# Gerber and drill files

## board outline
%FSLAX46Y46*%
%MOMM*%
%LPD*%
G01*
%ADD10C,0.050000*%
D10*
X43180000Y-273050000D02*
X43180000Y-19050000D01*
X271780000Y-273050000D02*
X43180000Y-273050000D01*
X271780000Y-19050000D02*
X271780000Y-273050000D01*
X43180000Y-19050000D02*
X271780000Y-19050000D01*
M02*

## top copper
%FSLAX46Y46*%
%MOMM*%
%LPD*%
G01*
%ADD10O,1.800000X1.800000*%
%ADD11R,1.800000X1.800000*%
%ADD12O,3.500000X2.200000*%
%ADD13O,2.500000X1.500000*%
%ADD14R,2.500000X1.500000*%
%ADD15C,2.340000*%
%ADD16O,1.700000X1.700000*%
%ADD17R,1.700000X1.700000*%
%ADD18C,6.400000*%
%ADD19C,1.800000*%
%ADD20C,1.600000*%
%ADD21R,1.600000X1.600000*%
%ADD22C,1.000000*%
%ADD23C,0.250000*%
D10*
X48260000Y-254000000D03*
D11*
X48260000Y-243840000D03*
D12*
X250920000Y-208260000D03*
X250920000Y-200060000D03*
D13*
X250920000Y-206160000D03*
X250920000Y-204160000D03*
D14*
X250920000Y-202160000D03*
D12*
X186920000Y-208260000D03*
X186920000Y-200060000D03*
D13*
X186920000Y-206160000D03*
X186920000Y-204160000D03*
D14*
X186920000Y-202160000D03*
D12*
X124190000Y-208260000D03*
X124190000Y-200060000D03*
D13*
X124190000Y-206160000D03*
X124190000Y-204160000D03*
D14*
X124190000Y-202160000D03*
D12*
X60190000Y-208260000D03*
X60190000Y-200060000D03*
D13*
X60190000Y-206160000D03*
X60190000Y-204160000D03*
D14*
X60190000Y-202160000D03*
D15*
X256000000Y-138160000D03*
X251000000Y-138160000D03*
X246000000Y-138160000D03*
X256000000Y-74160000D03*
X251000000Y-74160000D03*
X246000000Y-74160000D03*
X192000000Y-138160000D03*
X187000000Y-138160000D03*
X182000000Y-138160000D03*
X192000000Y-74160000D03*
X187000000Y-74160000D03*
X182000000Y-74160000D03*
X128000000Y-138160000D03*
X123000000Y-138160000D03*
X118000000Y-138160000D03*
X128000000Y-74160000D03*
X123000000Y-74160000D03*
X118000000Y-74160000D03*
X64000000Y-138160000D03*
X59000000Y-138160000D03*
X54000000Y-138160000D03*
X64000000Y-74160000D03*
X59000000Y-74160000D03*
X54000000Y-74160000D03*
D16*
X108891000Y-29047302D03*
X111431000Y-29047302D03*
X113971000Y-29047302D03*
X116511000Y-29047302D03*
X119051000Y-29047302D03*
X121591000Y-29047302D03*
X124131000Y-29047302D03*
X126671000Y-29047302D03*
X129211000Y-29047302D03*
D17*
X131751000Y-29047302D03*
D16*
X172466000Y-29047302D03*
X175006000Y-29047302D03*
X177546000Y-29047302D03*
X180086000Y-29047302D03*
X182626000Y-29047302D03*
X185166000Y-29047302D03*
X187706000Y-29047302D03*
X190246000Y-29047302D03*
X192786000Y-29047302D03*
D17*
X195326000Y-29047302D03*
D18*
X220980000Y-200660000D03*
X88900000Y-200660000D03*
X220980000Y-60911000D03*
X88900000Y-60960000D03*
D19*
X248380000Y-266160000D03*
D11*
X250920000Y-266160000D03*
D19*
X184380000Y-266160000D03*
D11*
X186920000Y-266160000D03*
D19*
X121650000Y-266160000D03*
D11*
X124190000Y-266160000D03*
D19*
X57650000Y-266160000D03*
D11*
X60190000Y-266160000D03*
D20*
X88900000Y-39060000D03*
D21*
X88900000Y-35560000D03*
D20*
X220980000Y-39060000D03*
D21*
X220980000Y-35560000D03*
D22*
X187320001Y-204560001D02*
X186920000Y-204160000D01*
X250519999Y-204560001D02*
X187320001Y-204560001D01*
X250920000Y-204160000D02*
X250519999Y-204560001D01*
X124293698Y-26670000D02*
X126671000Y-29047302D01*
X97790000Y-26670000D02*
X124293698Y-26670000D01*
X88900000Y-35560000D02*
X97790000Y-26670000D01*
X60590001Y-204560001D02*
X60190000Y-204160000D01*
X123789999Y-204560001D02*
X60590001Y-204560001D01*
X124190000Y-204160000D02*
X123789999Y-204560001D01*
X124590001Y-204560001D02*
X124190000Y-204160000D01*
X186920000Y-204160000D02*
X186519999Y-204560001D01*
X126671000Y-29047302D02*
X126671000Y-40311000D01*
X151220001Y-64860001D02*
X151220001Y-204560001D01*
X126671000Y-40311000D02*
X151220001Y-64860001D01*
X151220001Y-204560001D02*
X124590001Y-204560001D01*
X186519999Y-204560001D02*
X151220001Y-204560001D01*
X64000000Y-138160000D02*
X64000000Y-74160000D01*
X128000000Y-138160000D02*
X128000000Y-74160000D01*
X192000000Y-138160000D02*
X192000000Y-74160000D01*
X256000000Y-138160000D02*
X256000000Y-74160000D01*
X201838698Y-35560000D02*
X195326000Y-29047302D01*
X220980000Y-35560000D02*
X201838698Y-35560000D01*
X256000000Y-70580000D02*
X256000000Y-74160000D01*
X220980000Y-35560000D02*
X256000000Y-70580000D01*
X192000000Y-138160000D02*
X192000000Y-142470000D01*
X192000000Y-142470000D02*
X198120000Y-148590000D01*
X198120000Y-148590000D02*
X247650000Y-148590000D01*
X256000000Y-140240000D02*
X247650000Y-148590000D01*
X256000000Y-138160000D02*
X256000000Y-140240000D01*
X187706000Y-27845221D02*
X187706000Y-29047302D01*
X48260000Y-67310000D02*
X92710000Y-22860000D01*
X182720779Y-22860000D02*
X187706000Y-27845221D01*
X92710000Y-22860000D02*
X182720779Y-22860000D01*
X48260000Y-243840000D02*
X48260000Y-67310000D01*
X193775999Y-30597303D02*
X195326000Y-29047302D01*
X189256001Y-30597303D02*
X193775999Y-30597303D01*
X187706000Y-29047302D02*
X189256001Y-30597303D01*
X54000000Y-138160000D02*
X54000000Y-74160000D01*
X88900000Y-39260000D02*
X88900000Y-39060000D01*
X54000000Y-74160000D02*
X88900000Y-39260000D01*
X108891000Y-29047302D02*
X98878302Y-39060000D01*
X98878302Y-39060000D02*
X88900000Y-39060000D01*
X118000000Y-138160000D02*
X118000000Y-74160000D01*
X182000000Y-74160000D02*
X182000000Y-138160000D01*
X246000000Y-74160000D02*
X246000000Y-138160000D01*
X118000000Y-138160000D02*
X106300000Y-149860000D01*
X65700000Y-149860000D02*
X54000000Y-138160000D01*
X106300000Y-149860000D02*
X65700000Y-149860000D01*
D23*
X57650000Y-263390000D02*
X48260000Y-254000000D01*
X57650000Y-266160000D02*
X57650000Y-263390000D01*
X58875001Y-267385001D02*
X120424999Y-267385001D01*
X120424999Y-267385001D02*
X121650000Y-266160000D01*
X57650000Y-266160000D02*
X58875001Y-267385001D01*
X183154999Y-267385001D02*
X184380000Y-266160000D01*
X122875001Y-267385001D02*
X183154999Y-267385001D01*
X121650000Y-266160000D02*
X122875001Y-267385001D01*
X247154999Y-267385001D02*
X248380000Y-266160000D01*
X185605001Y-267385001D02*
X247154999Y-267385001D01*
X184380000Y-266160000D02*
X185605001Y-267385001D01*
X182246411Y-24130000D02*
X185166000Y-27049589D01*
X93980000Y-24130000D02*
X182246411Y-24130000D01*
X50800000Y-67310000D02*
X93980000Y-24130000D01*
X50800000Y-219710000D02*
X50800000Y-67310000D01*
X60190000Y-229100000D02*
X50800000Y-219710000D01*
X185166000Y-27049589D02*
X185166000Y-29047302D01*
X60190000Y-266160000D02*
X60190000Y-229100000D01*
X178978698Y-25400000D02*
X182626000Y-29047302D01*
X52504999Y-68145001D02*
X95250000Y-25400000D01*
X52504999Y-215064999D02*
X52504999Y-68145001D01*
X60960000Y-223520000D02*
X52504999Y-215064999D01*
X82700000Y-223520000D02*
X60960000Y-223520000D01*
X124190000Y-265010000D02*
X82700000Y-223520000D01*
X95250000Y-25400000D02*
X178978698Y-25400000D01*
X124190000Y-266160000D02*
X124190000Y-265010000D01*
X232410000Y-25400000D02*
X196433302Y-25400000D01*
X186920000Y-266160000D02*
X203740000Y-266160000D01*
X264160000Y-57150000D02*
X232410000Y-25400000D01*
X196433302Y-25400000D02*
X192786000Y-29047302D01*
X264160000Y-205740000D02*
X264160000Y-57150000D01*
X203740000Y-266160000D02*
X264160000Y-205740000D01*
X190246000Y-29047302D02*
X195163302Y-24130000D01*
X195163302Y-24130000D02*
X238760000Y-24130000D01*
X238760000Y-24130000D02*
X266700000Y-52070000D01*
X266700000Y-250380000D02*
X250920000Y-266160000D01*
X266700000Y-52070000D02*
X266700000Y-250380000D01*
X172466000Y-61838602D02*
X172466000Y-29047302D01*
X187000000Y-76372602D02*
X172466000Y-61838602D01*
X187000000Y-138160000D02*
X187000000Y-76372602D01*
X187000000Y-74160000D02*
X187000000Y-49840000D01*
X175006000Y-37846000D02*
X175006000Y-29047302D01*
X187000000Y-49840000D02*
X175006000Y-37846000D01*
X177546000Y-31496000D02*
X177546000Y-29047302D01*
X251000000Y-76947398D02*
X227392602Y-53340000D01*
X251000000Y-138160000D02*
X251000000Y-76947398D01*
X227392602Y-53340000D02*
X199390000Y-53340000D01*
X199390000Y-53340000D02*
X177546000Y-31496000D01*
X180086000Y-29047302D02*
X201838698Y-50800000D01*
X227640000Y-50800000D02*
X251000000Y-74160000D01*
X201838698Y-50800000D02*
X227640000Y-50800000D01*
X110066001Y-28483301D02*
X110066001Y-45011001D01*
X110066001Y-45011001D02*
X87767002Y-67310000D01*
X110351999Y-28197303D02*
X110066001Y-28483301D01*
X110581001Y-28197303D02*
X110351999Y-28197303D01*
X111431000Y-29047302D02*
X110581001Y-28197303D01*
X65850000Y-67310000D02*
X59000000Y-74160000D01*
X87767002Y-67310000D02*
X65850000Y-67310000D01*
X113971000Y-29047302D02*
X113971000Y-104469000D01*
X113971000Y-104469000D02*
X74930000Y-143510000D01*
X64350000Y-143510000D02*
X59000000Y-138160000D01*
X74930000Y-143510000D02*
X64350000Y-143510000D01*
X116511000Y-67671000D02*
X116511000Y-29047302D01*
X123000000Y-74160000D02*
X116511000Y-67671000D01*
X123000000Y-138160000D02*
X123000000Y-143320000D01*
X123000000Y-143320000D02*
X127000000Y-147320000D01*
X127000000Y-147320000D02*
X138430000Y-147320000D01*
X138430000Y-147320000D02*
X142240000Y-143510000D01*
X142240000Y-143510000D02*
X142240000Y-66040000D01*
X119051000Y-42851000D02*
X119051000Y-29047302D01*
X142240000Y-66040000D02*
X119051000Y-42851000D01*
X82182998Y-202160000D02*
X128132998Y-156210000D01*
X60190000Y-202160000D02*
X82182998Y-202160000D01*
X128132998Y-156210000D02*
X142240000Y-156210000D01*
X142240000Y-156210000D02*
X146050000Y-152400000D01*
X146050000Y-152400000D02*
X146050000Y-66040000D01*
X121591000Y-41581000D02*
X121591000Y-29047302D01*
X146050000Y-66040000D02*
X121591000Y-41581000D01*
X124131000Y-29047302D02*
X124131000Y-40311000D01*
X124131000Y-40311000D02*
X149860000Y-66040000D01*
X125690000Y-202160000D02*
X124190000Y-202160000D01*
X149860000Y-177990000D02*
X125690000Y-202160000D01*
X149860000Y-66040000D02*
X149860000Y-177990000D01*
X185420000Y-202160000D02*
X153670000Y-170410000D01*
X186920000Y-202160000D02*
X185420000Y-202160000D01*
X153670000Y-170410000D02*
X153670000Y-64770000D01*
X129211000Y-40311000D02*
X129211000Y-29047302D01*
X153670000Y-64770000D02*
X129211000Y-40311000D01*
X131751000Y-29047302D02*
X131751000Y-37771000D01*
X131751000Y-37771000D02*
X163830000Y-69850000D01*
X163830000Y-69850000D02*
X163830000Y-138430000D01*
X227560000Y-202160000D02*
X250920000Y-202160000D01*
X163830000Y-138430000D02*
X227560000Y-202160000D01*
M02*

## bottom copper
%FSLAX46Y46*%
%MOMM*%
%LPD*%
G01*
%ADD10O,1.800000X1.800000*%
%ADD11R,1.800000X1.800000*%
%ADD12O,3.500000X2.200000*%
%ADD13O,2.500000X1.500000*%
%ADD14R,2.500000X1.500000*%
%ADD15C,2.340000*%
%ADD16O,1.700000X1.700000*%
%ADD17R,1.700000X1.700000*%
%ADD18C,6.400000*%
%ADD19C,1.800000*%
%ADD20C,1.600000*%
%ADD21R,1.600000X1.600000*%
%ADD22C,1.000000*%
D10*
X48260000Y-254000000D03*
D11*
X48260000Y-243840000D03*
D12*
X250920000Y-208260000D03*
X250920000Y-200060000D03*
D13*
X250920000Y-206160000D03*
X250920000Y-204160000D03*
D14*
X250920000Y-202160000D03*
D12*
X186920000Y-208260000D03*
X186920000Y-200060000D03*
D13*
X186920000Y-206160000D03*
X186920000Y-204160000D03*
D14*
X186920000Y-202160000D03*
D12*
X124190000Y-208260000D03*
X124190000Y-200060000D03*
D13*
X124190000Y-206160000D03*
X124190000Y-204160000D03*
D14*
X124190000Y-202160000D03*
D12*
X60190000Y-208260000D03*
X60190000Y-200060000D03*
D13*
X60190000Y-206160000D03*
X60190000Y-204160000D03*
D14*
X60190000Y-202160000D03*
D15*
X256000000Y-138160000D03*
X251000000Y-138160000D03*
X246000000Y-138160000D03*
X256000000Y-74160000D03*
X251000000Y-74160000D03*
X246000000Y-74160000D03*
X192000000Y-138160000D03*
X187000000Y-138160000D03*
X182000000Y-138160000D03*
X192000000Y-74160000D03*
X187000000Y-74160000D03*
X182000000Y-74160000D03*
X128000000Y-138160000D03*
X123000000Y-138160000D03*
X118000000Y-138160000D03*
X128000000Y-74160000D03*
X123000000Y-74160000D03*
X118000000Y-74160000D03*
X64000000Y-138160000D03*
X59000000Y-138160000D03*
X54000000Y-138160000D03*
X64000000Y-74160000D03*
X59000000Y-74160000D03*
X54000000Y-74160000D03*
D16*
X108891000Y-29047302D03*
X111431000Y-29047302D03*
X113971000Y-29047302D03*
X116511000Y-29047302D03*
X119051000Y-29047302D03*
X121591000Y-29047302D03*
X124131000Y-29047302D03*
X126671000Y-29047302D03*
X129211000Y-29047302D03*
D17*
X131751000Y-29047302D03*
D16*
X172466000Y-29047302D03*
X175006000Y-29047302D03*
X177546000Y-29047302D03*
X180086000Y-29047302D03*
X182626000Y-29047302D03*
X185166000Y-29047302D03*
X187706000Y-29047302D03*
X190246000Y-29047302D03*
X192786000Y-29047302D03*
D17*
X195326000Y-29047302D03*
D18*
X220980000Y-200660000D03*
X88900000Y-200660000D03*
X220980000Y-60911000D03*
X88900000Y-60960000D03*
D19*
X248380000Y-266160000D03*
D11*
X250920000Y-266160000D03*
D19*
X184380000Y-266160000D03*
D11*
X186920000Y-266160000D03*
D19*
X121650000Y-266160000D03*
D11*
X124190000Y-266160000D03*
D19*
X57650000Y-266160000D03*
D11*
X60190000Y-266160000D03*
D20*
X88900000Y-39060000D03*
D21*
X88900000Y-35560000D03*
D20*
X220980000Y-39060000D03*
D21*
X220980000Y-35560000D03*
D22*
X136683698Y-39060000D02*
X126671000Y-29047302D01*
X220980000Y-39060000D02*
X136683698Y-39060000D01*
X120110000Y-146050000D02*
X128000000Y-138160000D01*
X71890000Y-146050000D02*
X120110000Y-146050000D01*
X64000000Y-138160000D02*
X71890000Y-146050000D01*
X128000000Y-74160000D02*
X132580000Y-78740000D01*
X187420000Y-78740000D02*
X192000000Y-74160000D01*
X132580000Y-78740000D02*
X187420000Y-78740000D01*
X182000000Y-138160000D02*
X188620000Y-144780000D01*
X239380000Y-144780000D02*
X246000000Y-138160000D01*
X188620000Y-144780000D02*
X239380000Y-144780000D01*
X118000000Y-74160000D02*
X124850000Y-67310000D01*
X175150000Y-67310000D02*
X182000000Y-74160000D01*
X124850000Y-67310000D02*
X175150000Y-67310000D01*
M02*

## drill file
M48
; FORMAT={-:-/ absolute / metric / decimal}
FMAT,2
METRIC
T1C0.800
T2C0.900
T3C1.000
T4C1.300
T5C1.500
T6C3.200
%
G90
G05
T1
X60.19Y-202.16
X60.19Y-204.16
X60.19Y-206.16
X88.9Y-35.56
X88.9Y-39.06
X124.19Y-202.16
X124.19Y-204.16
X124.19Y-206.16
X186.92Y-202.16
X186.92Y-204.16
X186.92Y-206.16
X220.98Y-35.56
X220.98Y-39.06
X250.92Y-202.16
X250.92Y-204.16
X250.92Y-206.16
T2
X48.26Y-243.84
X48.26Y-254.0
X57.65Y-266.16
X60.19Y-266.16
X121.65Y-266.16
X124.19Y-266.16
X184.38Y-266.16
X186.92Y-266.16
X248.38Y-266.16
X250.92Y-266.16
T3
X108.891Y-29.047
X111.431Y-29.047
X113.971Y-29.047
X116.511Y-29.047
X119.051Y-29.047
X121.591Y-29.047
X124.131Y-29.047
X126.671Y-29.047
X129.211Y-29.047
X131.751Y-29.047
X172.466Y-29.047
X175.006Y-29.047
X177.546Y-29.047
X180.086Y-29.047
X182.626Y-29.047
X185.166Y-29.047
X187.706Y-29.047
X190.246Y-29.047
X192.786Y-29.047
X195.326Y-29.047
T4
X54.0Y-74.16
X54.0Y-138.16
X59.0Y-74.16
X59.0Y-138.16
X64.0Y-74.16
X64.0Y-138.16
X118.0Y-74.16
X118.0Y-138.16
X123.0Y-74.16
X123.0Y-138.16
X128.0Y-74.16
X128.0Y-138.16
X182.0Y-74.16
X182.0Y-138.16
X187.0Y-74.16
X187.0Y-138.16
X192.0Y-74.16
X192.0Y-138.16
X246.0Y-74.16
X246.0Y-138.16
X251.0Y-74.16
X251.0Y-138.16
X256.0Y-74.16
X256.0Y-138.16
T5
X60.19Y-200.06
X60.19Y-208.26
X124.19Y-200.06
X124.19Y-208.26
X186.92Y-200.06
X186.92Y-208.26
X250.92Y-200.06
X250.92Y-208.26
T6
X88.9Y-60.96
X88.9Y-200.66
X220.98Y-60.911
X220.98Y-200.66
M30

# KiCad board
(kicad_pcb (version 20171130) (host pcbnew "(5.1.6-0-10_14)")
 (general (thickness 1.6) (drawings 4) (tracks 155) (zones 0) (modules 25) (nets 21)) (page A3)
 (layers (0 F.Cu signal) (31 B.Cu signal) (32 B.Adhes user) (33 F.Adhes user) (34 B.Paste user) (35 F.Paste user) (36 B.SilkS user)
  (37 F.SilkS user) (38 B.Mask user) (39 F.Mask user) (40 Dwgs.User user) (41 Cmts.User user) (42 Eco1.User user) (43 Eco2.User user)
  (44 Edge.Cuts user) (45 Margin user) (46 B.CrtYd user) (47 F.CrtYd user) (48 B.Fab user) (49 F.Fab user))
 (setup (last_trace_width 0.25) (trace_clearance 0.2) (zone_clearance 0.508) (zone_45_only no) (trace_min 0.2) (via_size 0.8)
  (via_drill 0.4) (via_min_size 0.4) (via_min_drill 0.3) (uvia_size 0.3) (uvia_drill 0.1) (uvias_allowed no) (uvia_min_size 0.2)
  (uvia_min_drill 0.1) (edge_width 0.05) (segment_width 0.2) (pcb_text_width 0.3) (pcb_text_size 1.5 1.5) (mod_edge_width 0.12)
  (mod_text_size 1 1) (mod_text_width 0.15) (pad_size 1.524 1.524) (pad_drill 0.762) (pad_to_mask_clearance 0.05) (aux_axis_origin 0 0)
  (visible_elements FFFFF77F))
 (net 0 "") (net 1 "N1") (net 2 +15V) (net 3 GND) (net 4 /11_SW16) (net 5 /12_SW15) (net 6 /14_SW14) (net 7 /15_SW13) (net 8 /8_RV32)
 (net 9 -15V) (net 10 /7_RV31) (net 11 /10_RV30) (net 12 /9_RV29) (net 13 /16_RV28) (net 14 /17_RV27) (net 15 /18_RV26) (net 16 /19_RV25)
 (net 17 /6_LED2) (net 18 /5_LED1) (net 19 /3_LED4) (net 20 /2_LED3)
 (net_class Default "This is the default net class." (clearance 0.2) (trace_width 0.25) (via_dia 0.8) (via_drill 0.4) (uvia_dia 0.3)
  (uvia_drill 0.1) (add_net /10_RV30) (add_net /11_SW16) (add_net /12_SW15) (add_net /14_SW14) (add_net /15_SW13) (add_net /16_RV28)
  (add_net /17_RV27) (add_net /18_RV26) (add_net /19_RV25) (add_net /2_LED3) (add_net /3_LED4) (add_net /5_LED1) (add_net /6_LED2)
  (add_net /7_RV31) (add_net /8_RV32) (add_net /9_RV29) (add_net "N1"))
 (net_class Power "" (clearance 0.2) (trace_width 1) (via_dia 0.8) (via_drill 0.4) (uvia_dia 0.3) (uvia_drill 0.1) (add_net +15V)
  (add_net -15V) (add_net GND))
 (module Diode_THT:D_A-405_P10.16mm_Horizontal (layer F.Cu) (at 48.26 243.84 270)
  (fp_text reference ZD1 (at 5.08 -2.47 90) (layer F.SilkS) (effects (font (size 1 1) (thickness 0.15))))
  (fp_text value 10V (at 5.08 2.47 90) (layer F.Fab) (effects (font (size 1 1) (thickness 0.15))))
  (pad 2 thru_hole oval (at 10.16 0 270) (size 1.8 1.8) (drill 0.9) (layers *.Cu *.Mask) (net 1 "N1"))
  (pad 1 thru_hole rect (at 0 0 270) (size 1.8 1.8) (drill 0.9) (layers *.Cu *.Mask) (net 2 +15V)))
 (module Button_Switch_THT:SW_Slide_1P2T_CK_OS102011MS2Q (layer F.Cu) (at 250.92 202.16 270)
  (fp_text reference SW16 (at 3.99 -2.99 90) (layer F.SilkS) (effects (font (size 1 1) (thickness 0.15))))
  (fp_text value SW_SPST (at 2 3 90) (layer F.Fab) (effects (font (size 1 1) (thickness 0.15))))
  (pad "" thru_hole oval (at 6.1 0 270) (size 2.2 3.5) (drill 1.5) (layers *.Cu *.Mask))
  (pad "" thru_hole oval (at -2.1 0 270) (size 2.2 3.5) (drill 1.5) (layers *.Cu *.Mask))
  (pad 3 thru_hole oval (at 4 0 270) (size 1.5 2.5) (drill 0.8) (layers *.Cu *.Mask))
  (pad 2 thru_hole oval (at 2 0 270) (size 1.5 2.5) (drill 0.8) (layers *.Cu *.Mask) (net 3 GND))
  (pad 1 thru_hole rect (at 0 0 270) (size 1.5 2.5) (drill 0.8) (layers *.Cu *.Mask) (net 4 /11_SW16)))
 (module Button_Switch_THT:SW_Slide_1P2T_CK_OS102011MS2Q (layer F.Cu) (at 186.92 202.16 270)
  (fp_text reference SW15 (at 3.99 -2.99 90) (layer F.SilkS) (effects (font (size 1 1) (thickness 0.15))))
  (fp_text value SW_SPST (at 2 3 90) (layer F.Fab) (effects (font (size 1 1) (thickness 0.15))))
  (pad "" thru_hole oval (at 6.1 0 270) (size 2.2 3.5) (drill 1.5) (layers *.Cu *.Mask))
  (pad "" thru_hole oval (at -2.1 0 270) (size 2.2 3.5) (drill 1.5) (layers *.Cu *.Mask))
  (pad 3 thru_hole oval (at 4 0 270) (size 1.5 2.5) (drill 0.8) (layers *.Cu *.Mask))
  (pad 2 thru_hole oval (at 2 0 270) (size 1.5 2.5) (drill 0.8) (layers *.Cu *.Mask) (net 3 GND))
  (pad 1 thru_hole rect (at 0 0 270) (size 1.5 2.5) (drill 0.8) (layers *.Cu *.Mask) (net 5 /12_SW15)))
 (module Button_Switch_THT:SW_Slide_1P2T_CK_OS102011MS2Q (layer F.Cu) (at 124.19 202.16 270)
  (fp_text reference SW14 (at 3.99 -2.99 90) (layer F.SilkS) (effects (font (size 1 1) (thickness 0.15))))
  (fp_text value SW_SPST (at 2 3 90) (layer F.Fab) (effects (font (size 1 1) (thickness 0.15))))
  (pad "" thru_hole oval (at 6.1 0 270) (size 2.2 3.5) (drill 1.5) (layers *.Cu *.Mask))
  (pad "" thru_hole oval (at -2.1 0 270) (size 2.2 3.5) (drill 1.5) (layers *.Cu *.Mask))
  (pad 3 thru_hole oval (at 4 0 270) (size 1.5 2.5) (drill 0.8) (layers *.Cu *.Mask))
  (pad 2 thru_hole oval (at 2 0 270) (size 1.5 2.5) (drill 0.8) (layers *.Cu *.Mask) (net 3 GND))
  (pad 1 thru_hole rect (at 0 0 270) (size 1.5 2.5) (drill 0.8) (layers *.Cu *.Mask) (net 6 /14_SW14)))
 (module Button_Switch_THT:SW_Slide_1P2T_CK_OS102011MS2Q (layer F.Cu) (at 60.19 202.16 270)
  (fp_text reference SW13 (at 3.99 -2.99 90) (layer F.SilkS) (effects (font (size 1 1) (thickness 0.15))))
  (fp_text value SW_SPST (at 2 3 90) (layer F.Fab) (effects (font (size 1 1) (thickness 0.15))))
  (pad "" thru_hole oval (at 6.1 0 270) (size 2.2 3.5) (drill 1.5) (layers *.Cu *.Mask))
  (pad "" thru_hole oval (at -2.1 0 270) (size 2.2 3.5) (drill 1.5) (layers *.Cu *.Mask))
  (pad 3 thru_hole oval (at 4 0 270) (size 1.5 2.5) (drill 0.8) (layers *.Cu *.Mask))
  (pad 2 thru_hole oval (at 2 0 270) (size 1.5 2.5) (drill 0.8) (layers *.Cu *.Mask) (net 3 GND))
  (pad 1 thru_hole rect (at 0 0 270) (size 1.5 2.5) (drill 0.8) (layers *.Cu *.Mask) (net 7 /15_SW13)))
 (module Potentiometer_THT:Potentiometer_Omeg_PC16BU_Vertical (layer F.Cu) (at 256 138.16 90)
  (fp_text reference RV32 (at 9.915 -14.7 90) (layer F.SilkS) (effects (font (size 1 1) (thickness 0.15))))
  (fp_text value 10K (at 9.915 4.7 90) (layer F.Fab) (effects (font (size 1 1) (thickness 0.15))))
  (pad 1 thru_hole circle (at 0 0 90) (size 2.34 2.34) (drill 1.3) (layers *.Cu *.Mask) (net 2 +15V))
  (pad 2 thru_hole circle (at 0 -5 90) (size 2.34 2.34) (drill 1.3) (layers *.Cu *.Mask) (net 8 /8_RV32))
  (pad 3 thru_hole circle (at 0 -10 90) (size 2.34 2.34) (drill 1.3) (layers *.Cu *.Mask) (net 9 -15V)))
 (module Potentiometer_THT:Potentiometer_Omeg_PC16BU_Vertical (layer F.Cu) (at 256 74.16 90)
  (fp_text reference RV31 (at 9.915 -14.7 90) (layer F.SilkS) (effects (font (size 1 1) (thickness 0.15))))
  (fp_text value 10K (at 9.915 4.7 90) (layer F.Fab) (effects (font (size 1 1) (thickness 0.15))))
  (pad 1 thru_hole circle (at 0 0 90) (size 2.34 2.34) (drill 1.3) (layers *.Cu *.Mask) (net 2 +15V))
  (pad 2 thru_hole circle (at 0 -5 90) (size 2.34 2.34) (drill 1.3) (layers *.Cu *.Mask) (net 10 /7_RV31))
  (pad 3 thru_hole circle (at 0 -10 90) (size 2.34 2.34) (drill 1.3) (layers *.Cu *.Mask) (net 9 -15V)))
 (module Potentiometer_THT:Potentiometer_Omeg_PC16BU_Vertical (layer F.Cu) (at 192 138.16 90)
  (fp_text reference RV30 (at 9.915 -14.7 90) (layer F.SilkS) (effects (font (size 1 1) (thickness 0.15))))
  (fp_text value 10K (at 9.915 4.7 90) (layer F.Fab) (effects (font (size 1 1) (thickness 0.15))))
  (pad 1 thru_hole circle (at 0 0 90) (size 2.34 2.34) (drill 1.3) (layers *.Cu *.Mask) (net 2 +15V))
  (pad 2 thru_hole circle (at 0 -5 90) (size 2.34 2.34) (drill 1.3) (layers *.Cu *.Mask) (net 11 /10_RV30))
  (pad 3 thru_hole circle (at 0 -10 90) (size 2.34 2.34) (drill 1.3) (layers *.Cu *.Mask) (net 9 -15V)))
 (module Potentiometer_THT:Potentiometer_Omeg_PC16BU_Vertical (layer F.Cu) (at 192 74.16 90)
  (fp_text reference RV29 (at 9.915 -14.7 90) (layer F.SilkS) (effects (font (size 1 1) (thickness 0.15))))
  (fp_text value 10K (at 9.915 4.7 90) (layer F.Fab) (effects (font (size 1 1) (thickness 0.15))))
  (pad 1 thru_hole circle (at 0 0 90) (size 2.34 2.34) (drill 1.3) (layers *.Cu *.Mask) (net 2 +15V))
  (pad 2 thru_hole circle (at 0 -5 90) (size 2.34 2.34) (drill 1.3) (layers *.Cu *.Mask) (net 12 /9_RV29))
  (pad 3 thru_hole circle (at 0 -10 90) (size 2.34 2.34) (drill 1.3) (layers *.Cu *.Mask) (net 9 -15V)))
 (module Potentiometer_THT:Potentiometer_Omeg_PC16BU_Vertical (layer F.Cu) (at 128 138.16 90)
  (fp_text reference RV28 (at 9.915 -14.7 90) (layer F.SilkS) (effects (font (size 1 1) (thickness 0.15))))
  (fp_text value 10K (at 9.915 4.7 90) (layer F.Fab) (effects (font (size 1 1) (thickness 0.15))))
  (pad 1 thru_hole circle (at 0 0 90) (size 2.34 2.34) (drill 1.3) (layers *.Cu *.Mask) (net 2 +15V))
  (pad 2 thru_hole circle (at 0 -5 90) (size 2.34 2.34) (drill 1.3) (layers *.Cu *.Mask) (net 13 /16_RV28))
  (pad 3 thru_hole circle (at 0 -10 90) (size 2.34 2.34) (drill 1.3) (layers *.Cu *.Mask) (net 9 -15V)))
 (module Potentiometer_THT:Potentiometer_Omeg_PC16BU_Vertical (layer F.Cu) (at 128 74.16 90)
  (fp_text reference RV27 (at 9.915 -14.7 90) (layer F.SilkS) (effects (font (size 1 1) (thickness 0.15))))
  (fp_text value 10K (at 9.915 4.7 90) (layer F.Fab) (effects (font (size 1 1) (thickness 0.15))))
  (pad 1 thru_hole circle (at 0 0 90) (size 2.34 2.34) (drill 1.3) (layers *.Cu *.Mask) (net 2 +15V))
  (pad 2 thru_hole circle (at 0 -5 90) (size 2.34 2.34) (drill 1.3) (layers *.Cu *.Mask) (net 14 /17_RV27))
  (pad 3 thru_hole circle (at 0 -10 90) (size 2.34 2.34) (drill 1.3) (layers *.Cu *.Mask) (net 9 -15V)))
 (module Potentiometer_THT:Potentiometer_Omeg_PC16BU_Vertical (layer F.Cu) (at 64 138.16 90)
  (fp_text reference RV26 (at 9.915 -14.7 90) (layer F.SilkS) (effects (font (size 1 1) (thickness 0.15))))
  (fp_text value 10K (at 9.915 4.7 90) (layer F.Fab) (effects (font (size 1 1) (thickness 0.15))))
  (pad 1 thru_hole circle (at 0 0 90) (size 2.34 2.34) (drill 1.3) (layers *.Cu *.Mask) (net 2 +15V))
  (pad 2 thru_hole circle (at 0 -5 90) (size 2.34 2.34) (drill 1.3) (layers *.Cu *.Mask) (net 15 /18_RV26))
  (pad 3 thru_hole circle (at 0 -10 90) (size 2.34 2.34) (drill 1.3) (layers *.Cu *.Mask) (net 9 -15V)))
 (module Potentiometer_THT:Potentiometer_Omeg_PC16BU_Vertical (layer F.Cu) (at 64 74.16 90)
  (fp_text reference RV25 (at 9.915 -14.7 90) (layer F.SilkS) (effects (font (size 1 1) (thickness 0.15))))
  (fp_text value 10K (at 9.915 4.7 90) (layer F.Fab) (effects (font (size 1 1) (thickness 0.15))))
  (pad 1 thru_hole circle (at 0 0 90) (size 2.34 2.34) (drill 1.3) (layers *.Cu *.Mask) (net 2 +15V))
  (pad 2 thru_hole circle (at 0 -5 90) (size 2.34 2.34) (drill 1.3) (layers *.Cu *.Mask) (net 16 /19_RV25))
  (pad 3 thru_hole circle (at 0 -10 90) (size 2.34 2.34) (drill 1.3) (layers *.Cu *.Mask) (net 9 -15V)))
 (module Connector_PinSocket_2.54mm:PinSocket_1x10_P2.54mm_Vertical (layer F.Cu) (at 131.751 29.047302 270)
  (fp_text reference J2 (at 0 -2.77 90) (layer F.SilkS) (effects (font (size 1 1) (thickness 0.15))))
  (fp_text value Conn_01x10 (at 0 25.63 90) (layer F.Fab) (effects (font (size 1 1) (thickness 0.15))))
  (pad 10 thru_hole oval (at 0 22.86 270) (size 1.7 1.7) (drill 1) (layers *.Cu *.Mask) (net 9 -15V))
  (pad 9 thru_hole oval (at 0 20.32 270) (size 1.7 1.7) (drill 1) (layers *.Cu *.Mask) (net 16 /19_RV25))
  (pad 8 thru_hole oval (at 0 17.78 270) (size 1.7 1.7) (drill 1) (layers *.Cu *.Mask) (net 15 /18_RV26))
  (pad 7 thru_hole oval (at 0 15.24 270) (size 1.7 1.7) (drill 1) (layers *.Cu *.Mask) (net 14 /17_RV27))
  (pad 6 thru_hole oval (at 0 12.7 270) (size 1.7 1.7) (drill 1) (layers *.Cu *.Mask) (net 13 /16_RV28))
  (pad 5 thru_hole oval (at 0 10.16 270) (size 1.7 1.7) (drill 1) (layers *.Cu *.Mask) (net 7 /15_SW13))
  (pad 4 thru_hole oval (at 0 7.62 270) (size 1.7 1.7) (drill 1) (layers *.Cu *.Mask) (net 6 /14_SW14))
  (pad 3 thru_hole oval (at 0 5.08 270) (size 1.7 1.7) (drill 1) (layers *.Cu *.Mask) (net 3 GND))
  (pad 2 thru_hole oval (at 0 2.54 270) (size 1.7 1.7) (drill 1) (layers *.Cu *.Mask) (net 5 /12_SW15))
  (pad 1 thru_hole rect (at 0 0 270) (size 1.7 1.7) (drill 1) (layers *.Cu *.Mask) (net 4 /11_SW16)))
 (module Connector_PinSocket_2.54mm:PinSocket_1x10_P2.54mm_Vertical (layer F.Cu) (at 195.326 29.047302 270)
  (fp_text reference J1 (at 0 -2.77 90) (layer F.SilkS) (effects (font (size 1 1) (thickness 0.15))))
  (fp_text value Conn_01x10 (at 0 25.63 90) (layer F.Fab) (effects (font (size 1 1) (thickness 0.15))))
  (pad 10 thru_hole oval (at 0 22.86 270) (size 1.7 1.7) (drill 1) (layers *.Cu *.Mask) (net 11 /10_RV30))
  (pad 9 thru_hole oval (at 0 20.32 270) (size 1.7 1.7) (drill 1) (layers *.Cu *.Mask) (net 12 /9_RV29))
  (pad 8 thru_hole oval (at 0 17.78 270) (size 1.7 1.7) (drill 1) (layers *.Cu *.Mask) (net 8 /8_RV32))
  (pad 7 thru_hole oval (at 0 15.24 270) (size 1.7 1.7) (drill 1) (layers *.Cu *.Mask) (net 10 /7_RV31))
  (pad 6 thru_hole oval (at 0 12.7 270) (size 1.7 1.7) (drill 1) (layers *.Cu *.Mask) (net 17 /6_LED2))
  (pad 5 thru_hole oval (at 0 10.16 270) (size 1.7 1.7) (drill 1) (layers *.Cu *.Mask) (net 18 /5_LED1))
  (pad 4 thru_hole oval (at 0 7.62 270) (size 1.7 1.7) (drill 1) (layers *.Cu *.Mask) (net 2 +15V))
  (pad 3 thru_hole oval (at 0 5.08 270) (size 1.7 1.7) (drill 1) (layers *.Cu *.Mask) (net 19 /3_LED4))
  (pad 2 thru_hole oval (at 0 2.54 270) (size 1.7 1.7) (drill 1) (layers *.Cu *.Mask) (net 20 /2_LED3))
  (pad 1 thru_hole rect (at 0 0 270) (size 1.7 1.7) (drill 1) (layers *.Cu *.Mask) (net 2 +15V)))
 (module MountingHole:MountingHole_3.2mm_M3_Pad (layer F.Cu) (at 220.98 200.66)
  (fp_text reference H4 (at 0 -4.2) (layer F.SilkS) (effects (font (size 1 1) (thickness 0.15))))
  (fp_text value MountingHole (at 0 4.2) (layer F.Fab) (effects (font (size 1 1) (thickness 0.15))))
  (pad 1 thru_hole circle (at 0 0) (size 6.4 6.4) (drill 3.2) (layers *.Cu *.Mask)))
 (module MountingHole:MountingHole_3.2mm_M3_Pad (layer F.Cu) (at 88.9 200.66)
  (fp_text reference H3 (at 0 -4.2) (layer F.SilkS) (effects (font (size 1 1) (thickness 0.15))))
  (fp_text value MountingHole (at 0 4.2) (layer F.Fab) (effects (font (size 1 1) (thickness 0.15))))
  (pad 1 thru_hole circle (at 0 0) (size 6.4 6.4) (drill 3.2) (layers *.Cu *.Mask)))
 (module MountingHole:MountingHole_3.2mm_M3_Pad (layer F.Cu) (at 220.98 60.911)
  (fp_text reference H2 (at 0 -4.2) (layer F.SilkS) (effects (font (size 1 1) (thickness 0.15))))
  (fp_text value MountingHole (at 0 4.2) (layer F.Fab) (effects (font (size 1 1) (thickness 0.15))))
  (pad 1 thru_hole circle (at 0 0) (size 6.4 6.4) (drill 3.2) (layers *.Cu *.Mask)))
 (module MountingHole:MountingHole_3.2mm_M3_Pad (layer F.Cu) (at 88.9 60.96)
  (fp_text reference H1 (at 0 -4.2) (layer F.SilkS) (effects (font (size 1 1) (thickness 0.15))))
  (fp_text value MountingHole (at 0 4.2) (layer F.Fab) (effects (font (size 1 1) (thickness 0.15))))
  (pad 1 thru_hole circle (at 0 0) (size 6.4 6.4) (drill 3.2) (layers *.Cu *.Mask)))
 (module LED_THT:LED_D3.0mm (layer F.Cu) (at 250.92 266.16 180)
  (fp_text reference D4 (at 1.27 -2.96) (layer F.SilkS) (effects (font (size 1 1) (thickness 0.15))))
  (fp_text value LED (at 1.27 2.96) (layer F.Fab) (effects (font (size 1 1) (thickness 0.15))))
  (pad 2 thru_hole circle (at 2.54 0 180) (size 1.8 1.8) (drill 0.9) (layers *.Cu *.Mask) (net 1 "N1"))
  (pad 1 thru_hole rect (at 0 0 180) (size 1.8 1.8) (drill 0.9) (layers *.Cu *.Mask) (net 19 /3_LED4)))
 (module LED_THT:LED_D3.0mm (layer F.Cu) (at 186.92 266.16 180)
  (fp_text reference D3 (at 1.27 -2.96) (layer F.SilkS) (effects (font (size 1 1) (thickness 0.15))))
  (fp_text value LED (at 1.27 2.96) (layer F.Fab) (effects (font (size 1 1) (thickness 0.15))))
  (pad 2 thru_hole circle (at 2.54 0 180) (size 1.8 1.8) (drill 0.9) (layers *.Cu *.Mask) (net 1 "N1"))
  (pad 1 thru_hole rect (at 0 0 180) (size 1.8 1.8) (drill 0.9) (layers *.Cu *.Mask) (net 20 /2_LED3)))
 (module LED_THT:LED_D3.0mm (layer F.Cu) (at 124.19 266.16 180)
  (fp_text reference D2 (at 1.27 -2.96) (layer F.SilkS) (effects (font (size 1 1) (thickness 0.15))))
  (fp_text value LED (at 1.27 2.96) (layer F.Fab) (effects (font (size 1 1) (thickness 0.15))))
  (pad 2 thru_hole circle (at 2.54 0 180) (size 1.8 1.8) (drill 0.9) (layers *.Cu *.Mask) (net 1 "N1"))
  (pad 1 thru_hole rect (at 0 0 180) (size 1.8 1.8) (drill 0.9) (layers *.Cu *.Mask) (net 17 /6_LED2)))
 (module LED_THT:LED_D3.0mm (layer F.Cu) (at 60.19 266.16 180)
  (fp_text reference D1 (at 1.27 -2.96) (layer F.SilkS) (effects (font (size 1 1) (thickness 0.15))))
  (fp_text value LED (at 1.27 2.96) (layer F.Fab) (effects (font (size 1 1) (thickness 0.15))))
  (pad 2 thru_hole circle (at 2.54 0 180) (size 1.8 1.8) (drill 0.9) (layers *.Cu *.Mask) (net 1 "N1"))
  (pad 1 thru_hole rect (at 0 0 180) (size 1.8 1.8) (drill 0.9) (layers *.Cu *.Mask) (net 18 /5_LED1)))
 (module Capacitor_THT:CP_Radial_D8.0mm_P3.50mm (layer F.Cu) (at 88.9 35.56 270)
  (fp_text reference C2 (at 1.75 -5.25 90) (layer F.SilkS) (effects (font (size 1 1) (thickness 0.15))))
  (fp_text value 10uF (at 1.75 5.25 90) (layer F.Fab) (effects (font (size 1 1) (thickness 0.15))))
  (pad 2 thru_hole circle (at 3.5 0 270) (size 1.6 1.6) (drill 0.8) (layers *.Cu *.Mask) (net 9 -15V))
  (pad 1 thru_hole rect (at 0 0 270) (size 1.6 1.6) (drill 0.8) (layers *.Cu *.Mask) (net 3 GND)))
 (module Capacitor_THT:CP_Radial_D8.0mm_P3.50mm (layer F.Cu) (at 220.98 35.56 270)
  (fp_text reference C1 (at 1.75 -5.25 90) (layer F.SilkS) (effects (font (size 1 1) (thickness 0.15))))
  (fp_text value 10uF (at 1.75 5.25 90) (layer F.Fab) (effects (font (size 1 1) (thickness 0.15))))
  (pad 2 thru_hole circle (at 3.5 0 270) (size 1.6 1.6) (drill 0.8) (layers *.Cu *.Mask) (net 3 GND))
  (pad 1 thru_hole rect (at 0 0 270) (size 1.6 1.6) (drill 0.8) (layers *.Cu *.Mask) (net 2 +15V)))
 (gr_line (start 43.18 273.05) (end 43.18 19.05) (layer Edge.Cuts) (width 0.05))
 (gr_line (start 271.78 273.05) (end 43.18 273.05) (layer Edge.Cuts) (width 0.05))
 (gr_line (start 271.78 19.05) (end 271.78 273.05) (layer Edge.Cuts) (width 0.05))
 (gr_line (start 43.18 19.05) (end 271.78 19.05) (layer Edge.Cuts) (width 0.05))
 (segment (start 136.683698 39.06) (end 126.671 29.047302) (width 1) (layer B.Cu) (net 3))
 (segment (start 220.98 39.06) (end 136.683698 39.06) (width 1) (layer B.Cu) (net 3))
 (segment (start 187.320001 204.560001) (end 186.92 204.16) (width 1) (layer F.Cu) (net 3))
 (segment (start 250.519999 204.560001) (end 187.320001 204.560001) (width 1) (layer F.Cu) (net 3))
 (segment (start 250.92 204.16) (end 250.519999 204.560001) (width 1) (layer F.Cu) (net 3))
 (segment (start 124.293698 26.67) (end 126.671 29.047302) (width 1) (layer F.Cu) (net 3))
 (segment (start 97.79 26.67) (end 124.293698 26.67) (width 1) (layer F.Cu) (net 3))
 (segment (start 88.9 35.56) (end 97.79 26.67) (width 1) (layer F.Cu) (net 3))
 (segment (start 60.590001 204.560001) (end 60.19 204.16) (width 1) (layer F.Cu) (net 3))
 (segment (start 123.789999 204.560001) (end 60.590001 204.560001) (width 1) (layer F.Cu) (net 3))
 (segment (start 124.19 204.16) (end 123.789999 204.560001) (width 1) (layer F.Cu) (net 3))
 (segment (start 124.590001 204.560001) (end 124.19 204.16) (width 1) (layer F.Cu) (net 3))
 (segment (start 186.92 204.16) (end 186.519999 204.560001) (width 1) (layer F.Cu) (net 3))
 (segment (start 126.671 29.047302) (end 126.671 40.311) (width 1) (layer F.Cu) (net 3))
 (segment (start 151.220001 64.860001) (end 151.220001 204.560001) (width 1) (layer F.Cu) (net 3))
 (segment (start 126.671 40.311) (end 151.220001 64.860001) (width 1) (layer F.Cu) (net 3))
 (segment (start 151.220001 204.560001) (end 124.590001 204.560001) (width 1) (layer F.Cu) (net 3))
 (segment (start 186.519999 204.560001) (end 151.220001 204.560001) (width 1) (layer F.Cu) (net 3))
 (segment (start 64 138.16) (end 64 74.16) (width 1) (layer F.Cu) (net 2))
 (segment (start 128 138.16) (end 128 74.16) (width 1) (layer F.Cu) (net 2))
 (segment (start 192 138.16) (end 192 74.16) (width 1) (layer F.Cu) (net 2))
 (segment (start 256 138.16) (end 256 74.16) (width 1) (layer F.Cu) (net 2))
 (segment (start 201.838698 35.56) (end 195.326 29.047302) (width 1) (layer F.Cu) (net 2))
 (segment (start 220.98 35.56) (end 201.838698 35.56) (width 1) (layer F.Cu) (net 2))
 (segment (start 256 70.58) (end 256 74.16) (width 1) (layer F.Cu) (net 2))
 (segment (start 220.98 35.56) (end 256 70.58) (width 1) (layer F.Cu) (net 2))
 (segment (start 192 138.16) (end 192 142.47) (width 1) (layer F.Cu) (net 2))
 (segment (start 192 142.47) (end 198.12 148.59) (width 1) (layer F.Cu) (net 2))
 (segment (start 198.12 148.59) (end 247.65 148.59) (width 1) (layer F.Cu) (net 2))
 (segment (start 256 140.24) (end 247.65 148.59) (width 1) (layer F.Cu) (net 2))
 (segment (start 256 138.16) (end 256 140.24) (width 1) (layer F.Cu) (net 2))
 (segment (start 120.11 146.05) (end 128 138.16) (width 1) (layer B.Cu) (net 2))
 (segment (start 71.89 146.05) (end 120.11 146.05) (width 1) (layer B.Cu) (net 2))
 (segment (start 64 138.16) (end 71.89 146.05) (width 1) (layer B.Cu) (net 2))
 (segment (start 187.706 27.845221) (end 187.706 29.047302) (width 1) (layer F.Cu) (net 2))
 (segment (start 48.26 67.31) (end 92.71 22.86) (width 1) (layer F.Cu) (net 2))
 (segment (start 182.720779 22.86) (end 187.706 27.845221) (width 1) (layer F.Cu) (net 2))
 (segment (start 92.71 22.86) (end 182.720779 22.86) (width 1) (layer F.Cu) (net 2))
 (segment (start 48.26 243.84) (end 48.26 67.31) (width 1) (layer F.Cu) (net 2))
 (segment (start 128 74.16) (end 132.58 78.74) (width 1) (layer B.Cu) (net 2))
 (segment (start 187.42 78.74) (end 192 74.16) (width 1) (layer B.Cu) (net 2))
 (segment (start 132.58 78.74) (end 187.42 78.74) (width 1) (layer B.Cu) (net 2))
 (segment (start 193.775999 30.597303) (end 195.326 29.047302) (width 1) (layer F.Cu) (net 2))
 (segment (start 189.256001 30.597303) (end 193.775999 30.597303) (width 1) (layer F.Cu) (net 2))
 (segment (start 187.706 29.047302) (end 189.256001 30.597303) (width 1) (layer F.Cu) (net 2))
 (segment (start 54 138.16) (end 54 74.16) (width 1) (layer F.Cu) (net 9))
 (segment (start 88.9 39.26) (end 88.9 39.06) (width 1) (layer F.Cu) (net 9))
 (segment (start 54 74.16) (end 88.9 39.26) (width 1) (layer F.Cu) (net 9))
 (segment (start 108.891 29.047302) (end 98.878302 39.06) (width 1) (layer F.Cu) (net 9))
 (segment (start 98.878302 39.06) (end 88.9 39.06) (width 1) (layer F.Cu) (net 9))
 (segment (start 118 138.16) (end 118 74.16) (width 1) (layer F.Cu) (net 9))
 (segment (start 182 74.16) (end 182 138.16) (width 1) (layer F.Cu) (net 9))
 (segment (start 246 74.16) (end 246 138.16) (width 1) (layer F.Cu) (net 9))
 (segment (start 182 138.16) (end 188.62 144.78) (width 1) (layer B.Cu) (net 9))
 (segment (start 239.38 144.78) (end 246 138.16) (width 1) (layer B.Cu) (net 9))
 (segment (start 188.62 144.78) (end 239.38 144.78) (width 1) (layer B.Cu) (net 9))
 (segment (start 118 138.16) (end 106.3 149.86) (width 1) (layer F.Cu) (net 9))
 (segment (start 65.7 149.86) (end 54 138.16) (width 1) (layer F.Cu) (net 9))
 (segment (start 106.3 149.86) (end 65.7 149.86) (width 1) (layer F.Cu) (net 9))
 (segment (start 118 74.16) (end 124.85 67.31) (width 1) (layer B.Cu) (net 9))
 (segment (start 175.15 67.31) (end 182 74.16) (width 1) (layer B.Cu) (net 9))
 (segment (start 124.85 67.31) (end 175.15 67.31) (width 1) (layer B.Cu) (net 9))
 (segment (start 57.65 263.39) (end 48.26 254) (width 0.25) (layer F.Cu) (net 1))
 (segment (start 57.65 266.16) (end 57.65 263.39) (width 0.25) (layer F.Cu) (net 1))
 (segment (start 58.875001 267.385001) (end 120.424999 267.385001) (width 0.25) (layer F.Cu) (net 1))
 (segment (start 120.424999 267.385001) (end 121.65 266.16) (width 0.25) (layer F.Cu) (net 1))
 (segment (start 57.65 266.16) (end 58.875001 267.385001) (width 0.25) (layer F.Cu) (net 1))
 (segment (start 183.154999 267.385001) (end 184.38 266.16) (width 0.25) (layer F.Cu) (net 1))
 (segment (start 122.875001 267.385001) (end 183.154999 267.385001) (width 0.25) (layer F.Cu) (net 1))
 (segment (start 121.65 266.16) (end 122.875001 267.385001) (width 0.25) (layer F.Cu) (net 1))
 (segment (start 247.154999 267.385001) (end 248.38 266.16) (width 0.25) (layer F.Cu) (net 1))
 (segment (start 185.605001 267.385001) (end 247.154999 267.385001) (width 0.25) (layer F.Cu) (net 1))
 (segment (start 184.38 266.16) (end 185.605001 267.385001) (width 0.25) (layer F.Cu) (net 1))
 (segment (start 182.246411 24.13) (end 185.166 27.049589) (width 0.25) (layer F.Cu) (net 18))
 (segment (start 93.98 24.13) (end 182.246411 24.13) (width 0.25) (layer F.Cu) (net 18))
 (segment (start 50.8 67.31) (end 93.98 24.13) (width 0.25) (layer F.Cu) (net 18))
 (segment (start 50.8 219.71) (end 50.8 67.31) (width 0.25) (layer F.Cu) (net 18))
 (segment (start 60.19 229.1) (end 50.8 219.71) (width 0.25) (layer F.Cu) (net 18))
 (segment (start 185.166 27.049589) (end 185.166 29.047302) (width 0.25) (layer F.Cu) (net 18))
 (segment (start 60.19 266.16) (end 60.19 229.1) (width 0.25) (layer F.Cu) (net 18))
 (segment (start 178.978698 25.4) (end 182.626 29.047302) (width 0.25) (layer F.Cu) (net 17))
 (segment (start 52.504999 68.145001) (end 95.25 25.4) (width 0.25) (layer F.Cu) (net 17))
 (segment (start 52.504999 215.064999) (end 52.504999 68.145001) (width 0.25) (layer F.Cu) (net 17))
 (segment (start 60.96 223.52) (end 52.504999 215.064999) (width 0.25) (layer F.Cu) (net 17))
 (segment (start 82.7 223.52) (end 60.96 223.52) (width 0.25) (layer F.Cu) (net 17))
 (segment (start 124.19 265.01) (end 82.7 223.52) (width 0.25) (layer F.Cu) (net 17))
 (segment (start 95.25 25.4) (end 178.978698 25.4) (width 0.25) (layer F.Cu) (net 17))
 (segment (start 124.19 266.16) (end 124.19 265.01) (width 0.25) (layer F.Cu) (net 17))
 (segment (start 232.41 25.4) (end 196.433302 25.4) (width 0.25) (layer F.Cu) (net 20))
 (segment (start 186.92 266.16) (end 203.74 266.16) (width 0.25) (layer F.Cu) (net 20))
 (segment (start 264.16 57.15) (end 232.41 25.4) (width 0.25) (layer F.Cu) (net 20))
 (segment (start 196.433302 25.4) (end 192.786 29.047302) (width 0.25) (layer F.Cu) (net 20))
 (segment (start 264.16 205.74) (end 264.16 57.15) (width 0.25) (layer F.Cu) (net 20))
 (segment (start 203.74 266.16) (end 264.16 205.74) (width 0.25) (layer F.Cu) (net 20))
 (segment (start 190.246 29.047302) (end 195.163302 24.13) (width 0.25) (layer F.Cu) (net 19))
 (segment (start 195.163302 24.13) (end 238.76 24.13) (width 0.25) (layer F.Cu) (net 19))
 (segment (start 238.76 24.13) (end 266.7 52.07) (width 0.25) (layer F.Cu) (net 19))
 (segment (start 266.7 250.38) (end 250.92 266.16) (width 0.25) (layer F.Cu) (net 19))
 (segment (start 266.7 52.07) (end 266.7 250.38) (width 0.25) (layer F.Cu) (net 19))
 (segment (start 172.466 61.838602) (end 172.466 29.047302) (width 0.25) (layer F.Cu) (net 11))
 (segment (start 187 76.372602) (end 172.466 61.838602) (width 0.25) (layer F.Cu) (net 11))
 (segment (start 187 138.16) (end 187 76.372602) (width 0.25) (layer F.Cu) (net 11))
 (segment (start 187 74.16) (end 187 49.84) (width 0.25) (layer F.Cu) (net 12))
 (segment (start 175.006 37.846) (end 175.006 29.047302) (width 0.25) (layer F.Cu) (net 12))
 (segment (start 187 49.84) (end 175.006 37.846) (width 0.25) (layer F.Cu) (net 12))
 (segment (start 177.546 31.496) (end 177.546 29.047302) (width 0.25) (layer F.Cu) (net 8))
 (segment (start 251 76.947398) (end 227.392602 53.34) (width 0.25) (layer F.Cu) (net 8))
 (segment (start 251 138.16) (end 251 76.947398) (width 0.25) (layer F.Cu) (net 8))
 (segment (start 227.392602 53.34) (end 199.39 53.34) (width 0.25) (layer F.Cu) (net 8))
 (segment (start 199.39 53.34) (end 177.546 31.496) (width 0.25) (layer F.Cu) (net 8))
 (segment (start 180.086 29.047302) (end 201.838698 50.8) (width 0.25) (layer F.Cu) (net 10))
 (segment (start 227.64 50.8) (end 251 74.16) (width 0.25) (layer F.Cu) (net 10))
 (segment (start 201.838698 50.8) (end 227.64 50.8) (width 0.25) (layer F.Cu) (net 10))
 (segment (start 110.066001 28.483301) (end 110.066001 45.011001) (width 0.25) (layer F.Cu) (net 16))
 (segment (start 110.066001 45.011001) (end 87.767002 67.31) (width 0.25) (layer F.Cu) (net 16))
 (segment (start 110.351999 28.197303) (end 110.066001 28.483301) (width 0.25) (layer F.Cu) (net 16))
 (segment (start 110.581001 28.197303) (end 110.351999 28.197303) (width 0.25) (layer F.Cu) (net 16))
 (segment (start 111.431 29.047302) (end 110.581001 28.197303) (width 0.25) (layer F.Cu) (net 16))
 (segment (start 65.85 67.31) (end 59 74.16) (width 0.25) (layer F.Cu) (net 16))
 (segment (start 87.767002 67.31) (end 65.85 67.31) (width 0.25) (layer F.Cu) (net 16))
 (segment (start 113.971 29.047302) (end 113.971 104.469) (width 0.25) (layer F.Cu) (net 15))
 (segment (start 113.971 104.469) (end 74.93 143.51) (width 0.25) (layer F.Cu) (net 15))
 (segment (start 64.35 143.51) (end 59 138.16) (width 0.25) (layer F.Cu) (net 15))
 (segment (start 74.93 143.51) (end 64.35 143.51) (width 0.25) (layer F.Cu) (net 15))
 (segment (start 116.511 67.671) (end 116.511 29.047302) (width 0.25) (layer F.Cu) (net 14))
 (segment (start 123 74.16) (end 116.511 67.671) (width 0.25) (layer F.Cu) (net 14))
 (segment (start 123 138.16) (end 123 143.32) (width 0.25) (layer F.Cu) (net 13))
 (segment (start 123 143.32) (end 127 147.32) (width 0.25) (layer F.Cu) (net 13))
 (segment (start 127 147.32) (end 138.43 147.32) (width 0.25) (layer F.Cu) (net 13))
 (segment (start 138.43 147.32) (end 142.24 143.51) (width 0.25) (layer F.Cu) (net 13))
 (segment (start 142.24 143.51) (end 142.24 66.04) (width 0.25) (layer F.Cu) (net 13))
 (segment (start 119.051 42.851) (end 119.051 29.047302) (width 0.25) (layer F.Cu) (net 13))
 (segment (start 142.24 66.04) (end 119.051 42.851) (width 0.25) (layer F.Cu) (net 13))
 (segment (start 82.182998 202.16) (end 128.132998 156.21) (width 0.25) (layer F.Cu) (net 7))
 (segment (start 60.19 202.16) (end 82.182998 202.16) (width 0.25) (layer F.Cu) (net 7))
 (segment (start 128.132998 156.21) (end 142.24 156.21) (width 0.25) (layer F.Cu) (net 7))
 (segment (start 142.24 156.21) (end 146.05 152.4) (width 0.25) (layer F.Cu) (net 7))
 (segment (start 146.05 152.4) (end 146.05 66.04) (width 0.25) (layer F.Cu) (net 7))
 (segment (start 121.591 41.581) (end 121.591 29.047302) (width 0.25) (layer F.Cu) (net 7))
 (segment (start 146.05 66.04) (end 121.591 41.581) (width 0.25) (layer F.Cu) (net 7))
 (segment (start 124.131 29.047302) (end 124.131 40.311) (width 0.25) (layer F.Cu) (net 6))
 (segment (start 124.131 40.311) (end 149.86 66.04) (width 0.25) (layer F.Cu) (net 6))
 (segment (start 125.69 202.16) (end 124.19 202.16) (width 0.25) (layer F.Cu) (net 6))
 (segment (start 149.86 177.99) (end 125.69 202.16) (width 0.25) (layer F.Cu) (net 6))
 (segment (start 149.86 66.04) (end 149.86 177.99) (width 0.25) (layer F.Cu) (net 6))
 (segment (start 185.42 202.16) (end 153.67 170.41) (width 0.25) (layer F.Cu) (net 5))
 (segment (start 186.92 202.16) (end 185.42 202.16) (width 0.25) (layer F.Cu) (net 5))
 (segment (start 153.67 170.41) (end 153.67 64.77) (width 0.25) (layer F.Cu) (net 5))
 (segment (start 129.211 40.311) (end 129.211 29.047302) (width 0.25) (layer F.Cu) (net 5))
 (segment (start 153.67 64.77) (end 129.211 40.311) (width 0.25) (layer F.Cu) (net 5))
 (segment (start 131.751 29.047302) (end 131.751 37.771) (width 0.25) (layer F.Cu) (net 4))
 (segment (start 131.751 37.771) (end 163.83 69.85) (width 0.25) (layer F.Cu) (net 4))
 (segment (start 163.83 69.85) (end 163.83 138.43) (width 0.25) (layer F.Cu) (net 4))
 (segment (start 227.56 202.16) (end 250.92 202.16) (width 0.25) (layer F.Cu) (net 4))
 (segment (start 163.83 138.43) (end 227.56 202.16) (width 0.25) (layer F.Cu) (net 4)))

